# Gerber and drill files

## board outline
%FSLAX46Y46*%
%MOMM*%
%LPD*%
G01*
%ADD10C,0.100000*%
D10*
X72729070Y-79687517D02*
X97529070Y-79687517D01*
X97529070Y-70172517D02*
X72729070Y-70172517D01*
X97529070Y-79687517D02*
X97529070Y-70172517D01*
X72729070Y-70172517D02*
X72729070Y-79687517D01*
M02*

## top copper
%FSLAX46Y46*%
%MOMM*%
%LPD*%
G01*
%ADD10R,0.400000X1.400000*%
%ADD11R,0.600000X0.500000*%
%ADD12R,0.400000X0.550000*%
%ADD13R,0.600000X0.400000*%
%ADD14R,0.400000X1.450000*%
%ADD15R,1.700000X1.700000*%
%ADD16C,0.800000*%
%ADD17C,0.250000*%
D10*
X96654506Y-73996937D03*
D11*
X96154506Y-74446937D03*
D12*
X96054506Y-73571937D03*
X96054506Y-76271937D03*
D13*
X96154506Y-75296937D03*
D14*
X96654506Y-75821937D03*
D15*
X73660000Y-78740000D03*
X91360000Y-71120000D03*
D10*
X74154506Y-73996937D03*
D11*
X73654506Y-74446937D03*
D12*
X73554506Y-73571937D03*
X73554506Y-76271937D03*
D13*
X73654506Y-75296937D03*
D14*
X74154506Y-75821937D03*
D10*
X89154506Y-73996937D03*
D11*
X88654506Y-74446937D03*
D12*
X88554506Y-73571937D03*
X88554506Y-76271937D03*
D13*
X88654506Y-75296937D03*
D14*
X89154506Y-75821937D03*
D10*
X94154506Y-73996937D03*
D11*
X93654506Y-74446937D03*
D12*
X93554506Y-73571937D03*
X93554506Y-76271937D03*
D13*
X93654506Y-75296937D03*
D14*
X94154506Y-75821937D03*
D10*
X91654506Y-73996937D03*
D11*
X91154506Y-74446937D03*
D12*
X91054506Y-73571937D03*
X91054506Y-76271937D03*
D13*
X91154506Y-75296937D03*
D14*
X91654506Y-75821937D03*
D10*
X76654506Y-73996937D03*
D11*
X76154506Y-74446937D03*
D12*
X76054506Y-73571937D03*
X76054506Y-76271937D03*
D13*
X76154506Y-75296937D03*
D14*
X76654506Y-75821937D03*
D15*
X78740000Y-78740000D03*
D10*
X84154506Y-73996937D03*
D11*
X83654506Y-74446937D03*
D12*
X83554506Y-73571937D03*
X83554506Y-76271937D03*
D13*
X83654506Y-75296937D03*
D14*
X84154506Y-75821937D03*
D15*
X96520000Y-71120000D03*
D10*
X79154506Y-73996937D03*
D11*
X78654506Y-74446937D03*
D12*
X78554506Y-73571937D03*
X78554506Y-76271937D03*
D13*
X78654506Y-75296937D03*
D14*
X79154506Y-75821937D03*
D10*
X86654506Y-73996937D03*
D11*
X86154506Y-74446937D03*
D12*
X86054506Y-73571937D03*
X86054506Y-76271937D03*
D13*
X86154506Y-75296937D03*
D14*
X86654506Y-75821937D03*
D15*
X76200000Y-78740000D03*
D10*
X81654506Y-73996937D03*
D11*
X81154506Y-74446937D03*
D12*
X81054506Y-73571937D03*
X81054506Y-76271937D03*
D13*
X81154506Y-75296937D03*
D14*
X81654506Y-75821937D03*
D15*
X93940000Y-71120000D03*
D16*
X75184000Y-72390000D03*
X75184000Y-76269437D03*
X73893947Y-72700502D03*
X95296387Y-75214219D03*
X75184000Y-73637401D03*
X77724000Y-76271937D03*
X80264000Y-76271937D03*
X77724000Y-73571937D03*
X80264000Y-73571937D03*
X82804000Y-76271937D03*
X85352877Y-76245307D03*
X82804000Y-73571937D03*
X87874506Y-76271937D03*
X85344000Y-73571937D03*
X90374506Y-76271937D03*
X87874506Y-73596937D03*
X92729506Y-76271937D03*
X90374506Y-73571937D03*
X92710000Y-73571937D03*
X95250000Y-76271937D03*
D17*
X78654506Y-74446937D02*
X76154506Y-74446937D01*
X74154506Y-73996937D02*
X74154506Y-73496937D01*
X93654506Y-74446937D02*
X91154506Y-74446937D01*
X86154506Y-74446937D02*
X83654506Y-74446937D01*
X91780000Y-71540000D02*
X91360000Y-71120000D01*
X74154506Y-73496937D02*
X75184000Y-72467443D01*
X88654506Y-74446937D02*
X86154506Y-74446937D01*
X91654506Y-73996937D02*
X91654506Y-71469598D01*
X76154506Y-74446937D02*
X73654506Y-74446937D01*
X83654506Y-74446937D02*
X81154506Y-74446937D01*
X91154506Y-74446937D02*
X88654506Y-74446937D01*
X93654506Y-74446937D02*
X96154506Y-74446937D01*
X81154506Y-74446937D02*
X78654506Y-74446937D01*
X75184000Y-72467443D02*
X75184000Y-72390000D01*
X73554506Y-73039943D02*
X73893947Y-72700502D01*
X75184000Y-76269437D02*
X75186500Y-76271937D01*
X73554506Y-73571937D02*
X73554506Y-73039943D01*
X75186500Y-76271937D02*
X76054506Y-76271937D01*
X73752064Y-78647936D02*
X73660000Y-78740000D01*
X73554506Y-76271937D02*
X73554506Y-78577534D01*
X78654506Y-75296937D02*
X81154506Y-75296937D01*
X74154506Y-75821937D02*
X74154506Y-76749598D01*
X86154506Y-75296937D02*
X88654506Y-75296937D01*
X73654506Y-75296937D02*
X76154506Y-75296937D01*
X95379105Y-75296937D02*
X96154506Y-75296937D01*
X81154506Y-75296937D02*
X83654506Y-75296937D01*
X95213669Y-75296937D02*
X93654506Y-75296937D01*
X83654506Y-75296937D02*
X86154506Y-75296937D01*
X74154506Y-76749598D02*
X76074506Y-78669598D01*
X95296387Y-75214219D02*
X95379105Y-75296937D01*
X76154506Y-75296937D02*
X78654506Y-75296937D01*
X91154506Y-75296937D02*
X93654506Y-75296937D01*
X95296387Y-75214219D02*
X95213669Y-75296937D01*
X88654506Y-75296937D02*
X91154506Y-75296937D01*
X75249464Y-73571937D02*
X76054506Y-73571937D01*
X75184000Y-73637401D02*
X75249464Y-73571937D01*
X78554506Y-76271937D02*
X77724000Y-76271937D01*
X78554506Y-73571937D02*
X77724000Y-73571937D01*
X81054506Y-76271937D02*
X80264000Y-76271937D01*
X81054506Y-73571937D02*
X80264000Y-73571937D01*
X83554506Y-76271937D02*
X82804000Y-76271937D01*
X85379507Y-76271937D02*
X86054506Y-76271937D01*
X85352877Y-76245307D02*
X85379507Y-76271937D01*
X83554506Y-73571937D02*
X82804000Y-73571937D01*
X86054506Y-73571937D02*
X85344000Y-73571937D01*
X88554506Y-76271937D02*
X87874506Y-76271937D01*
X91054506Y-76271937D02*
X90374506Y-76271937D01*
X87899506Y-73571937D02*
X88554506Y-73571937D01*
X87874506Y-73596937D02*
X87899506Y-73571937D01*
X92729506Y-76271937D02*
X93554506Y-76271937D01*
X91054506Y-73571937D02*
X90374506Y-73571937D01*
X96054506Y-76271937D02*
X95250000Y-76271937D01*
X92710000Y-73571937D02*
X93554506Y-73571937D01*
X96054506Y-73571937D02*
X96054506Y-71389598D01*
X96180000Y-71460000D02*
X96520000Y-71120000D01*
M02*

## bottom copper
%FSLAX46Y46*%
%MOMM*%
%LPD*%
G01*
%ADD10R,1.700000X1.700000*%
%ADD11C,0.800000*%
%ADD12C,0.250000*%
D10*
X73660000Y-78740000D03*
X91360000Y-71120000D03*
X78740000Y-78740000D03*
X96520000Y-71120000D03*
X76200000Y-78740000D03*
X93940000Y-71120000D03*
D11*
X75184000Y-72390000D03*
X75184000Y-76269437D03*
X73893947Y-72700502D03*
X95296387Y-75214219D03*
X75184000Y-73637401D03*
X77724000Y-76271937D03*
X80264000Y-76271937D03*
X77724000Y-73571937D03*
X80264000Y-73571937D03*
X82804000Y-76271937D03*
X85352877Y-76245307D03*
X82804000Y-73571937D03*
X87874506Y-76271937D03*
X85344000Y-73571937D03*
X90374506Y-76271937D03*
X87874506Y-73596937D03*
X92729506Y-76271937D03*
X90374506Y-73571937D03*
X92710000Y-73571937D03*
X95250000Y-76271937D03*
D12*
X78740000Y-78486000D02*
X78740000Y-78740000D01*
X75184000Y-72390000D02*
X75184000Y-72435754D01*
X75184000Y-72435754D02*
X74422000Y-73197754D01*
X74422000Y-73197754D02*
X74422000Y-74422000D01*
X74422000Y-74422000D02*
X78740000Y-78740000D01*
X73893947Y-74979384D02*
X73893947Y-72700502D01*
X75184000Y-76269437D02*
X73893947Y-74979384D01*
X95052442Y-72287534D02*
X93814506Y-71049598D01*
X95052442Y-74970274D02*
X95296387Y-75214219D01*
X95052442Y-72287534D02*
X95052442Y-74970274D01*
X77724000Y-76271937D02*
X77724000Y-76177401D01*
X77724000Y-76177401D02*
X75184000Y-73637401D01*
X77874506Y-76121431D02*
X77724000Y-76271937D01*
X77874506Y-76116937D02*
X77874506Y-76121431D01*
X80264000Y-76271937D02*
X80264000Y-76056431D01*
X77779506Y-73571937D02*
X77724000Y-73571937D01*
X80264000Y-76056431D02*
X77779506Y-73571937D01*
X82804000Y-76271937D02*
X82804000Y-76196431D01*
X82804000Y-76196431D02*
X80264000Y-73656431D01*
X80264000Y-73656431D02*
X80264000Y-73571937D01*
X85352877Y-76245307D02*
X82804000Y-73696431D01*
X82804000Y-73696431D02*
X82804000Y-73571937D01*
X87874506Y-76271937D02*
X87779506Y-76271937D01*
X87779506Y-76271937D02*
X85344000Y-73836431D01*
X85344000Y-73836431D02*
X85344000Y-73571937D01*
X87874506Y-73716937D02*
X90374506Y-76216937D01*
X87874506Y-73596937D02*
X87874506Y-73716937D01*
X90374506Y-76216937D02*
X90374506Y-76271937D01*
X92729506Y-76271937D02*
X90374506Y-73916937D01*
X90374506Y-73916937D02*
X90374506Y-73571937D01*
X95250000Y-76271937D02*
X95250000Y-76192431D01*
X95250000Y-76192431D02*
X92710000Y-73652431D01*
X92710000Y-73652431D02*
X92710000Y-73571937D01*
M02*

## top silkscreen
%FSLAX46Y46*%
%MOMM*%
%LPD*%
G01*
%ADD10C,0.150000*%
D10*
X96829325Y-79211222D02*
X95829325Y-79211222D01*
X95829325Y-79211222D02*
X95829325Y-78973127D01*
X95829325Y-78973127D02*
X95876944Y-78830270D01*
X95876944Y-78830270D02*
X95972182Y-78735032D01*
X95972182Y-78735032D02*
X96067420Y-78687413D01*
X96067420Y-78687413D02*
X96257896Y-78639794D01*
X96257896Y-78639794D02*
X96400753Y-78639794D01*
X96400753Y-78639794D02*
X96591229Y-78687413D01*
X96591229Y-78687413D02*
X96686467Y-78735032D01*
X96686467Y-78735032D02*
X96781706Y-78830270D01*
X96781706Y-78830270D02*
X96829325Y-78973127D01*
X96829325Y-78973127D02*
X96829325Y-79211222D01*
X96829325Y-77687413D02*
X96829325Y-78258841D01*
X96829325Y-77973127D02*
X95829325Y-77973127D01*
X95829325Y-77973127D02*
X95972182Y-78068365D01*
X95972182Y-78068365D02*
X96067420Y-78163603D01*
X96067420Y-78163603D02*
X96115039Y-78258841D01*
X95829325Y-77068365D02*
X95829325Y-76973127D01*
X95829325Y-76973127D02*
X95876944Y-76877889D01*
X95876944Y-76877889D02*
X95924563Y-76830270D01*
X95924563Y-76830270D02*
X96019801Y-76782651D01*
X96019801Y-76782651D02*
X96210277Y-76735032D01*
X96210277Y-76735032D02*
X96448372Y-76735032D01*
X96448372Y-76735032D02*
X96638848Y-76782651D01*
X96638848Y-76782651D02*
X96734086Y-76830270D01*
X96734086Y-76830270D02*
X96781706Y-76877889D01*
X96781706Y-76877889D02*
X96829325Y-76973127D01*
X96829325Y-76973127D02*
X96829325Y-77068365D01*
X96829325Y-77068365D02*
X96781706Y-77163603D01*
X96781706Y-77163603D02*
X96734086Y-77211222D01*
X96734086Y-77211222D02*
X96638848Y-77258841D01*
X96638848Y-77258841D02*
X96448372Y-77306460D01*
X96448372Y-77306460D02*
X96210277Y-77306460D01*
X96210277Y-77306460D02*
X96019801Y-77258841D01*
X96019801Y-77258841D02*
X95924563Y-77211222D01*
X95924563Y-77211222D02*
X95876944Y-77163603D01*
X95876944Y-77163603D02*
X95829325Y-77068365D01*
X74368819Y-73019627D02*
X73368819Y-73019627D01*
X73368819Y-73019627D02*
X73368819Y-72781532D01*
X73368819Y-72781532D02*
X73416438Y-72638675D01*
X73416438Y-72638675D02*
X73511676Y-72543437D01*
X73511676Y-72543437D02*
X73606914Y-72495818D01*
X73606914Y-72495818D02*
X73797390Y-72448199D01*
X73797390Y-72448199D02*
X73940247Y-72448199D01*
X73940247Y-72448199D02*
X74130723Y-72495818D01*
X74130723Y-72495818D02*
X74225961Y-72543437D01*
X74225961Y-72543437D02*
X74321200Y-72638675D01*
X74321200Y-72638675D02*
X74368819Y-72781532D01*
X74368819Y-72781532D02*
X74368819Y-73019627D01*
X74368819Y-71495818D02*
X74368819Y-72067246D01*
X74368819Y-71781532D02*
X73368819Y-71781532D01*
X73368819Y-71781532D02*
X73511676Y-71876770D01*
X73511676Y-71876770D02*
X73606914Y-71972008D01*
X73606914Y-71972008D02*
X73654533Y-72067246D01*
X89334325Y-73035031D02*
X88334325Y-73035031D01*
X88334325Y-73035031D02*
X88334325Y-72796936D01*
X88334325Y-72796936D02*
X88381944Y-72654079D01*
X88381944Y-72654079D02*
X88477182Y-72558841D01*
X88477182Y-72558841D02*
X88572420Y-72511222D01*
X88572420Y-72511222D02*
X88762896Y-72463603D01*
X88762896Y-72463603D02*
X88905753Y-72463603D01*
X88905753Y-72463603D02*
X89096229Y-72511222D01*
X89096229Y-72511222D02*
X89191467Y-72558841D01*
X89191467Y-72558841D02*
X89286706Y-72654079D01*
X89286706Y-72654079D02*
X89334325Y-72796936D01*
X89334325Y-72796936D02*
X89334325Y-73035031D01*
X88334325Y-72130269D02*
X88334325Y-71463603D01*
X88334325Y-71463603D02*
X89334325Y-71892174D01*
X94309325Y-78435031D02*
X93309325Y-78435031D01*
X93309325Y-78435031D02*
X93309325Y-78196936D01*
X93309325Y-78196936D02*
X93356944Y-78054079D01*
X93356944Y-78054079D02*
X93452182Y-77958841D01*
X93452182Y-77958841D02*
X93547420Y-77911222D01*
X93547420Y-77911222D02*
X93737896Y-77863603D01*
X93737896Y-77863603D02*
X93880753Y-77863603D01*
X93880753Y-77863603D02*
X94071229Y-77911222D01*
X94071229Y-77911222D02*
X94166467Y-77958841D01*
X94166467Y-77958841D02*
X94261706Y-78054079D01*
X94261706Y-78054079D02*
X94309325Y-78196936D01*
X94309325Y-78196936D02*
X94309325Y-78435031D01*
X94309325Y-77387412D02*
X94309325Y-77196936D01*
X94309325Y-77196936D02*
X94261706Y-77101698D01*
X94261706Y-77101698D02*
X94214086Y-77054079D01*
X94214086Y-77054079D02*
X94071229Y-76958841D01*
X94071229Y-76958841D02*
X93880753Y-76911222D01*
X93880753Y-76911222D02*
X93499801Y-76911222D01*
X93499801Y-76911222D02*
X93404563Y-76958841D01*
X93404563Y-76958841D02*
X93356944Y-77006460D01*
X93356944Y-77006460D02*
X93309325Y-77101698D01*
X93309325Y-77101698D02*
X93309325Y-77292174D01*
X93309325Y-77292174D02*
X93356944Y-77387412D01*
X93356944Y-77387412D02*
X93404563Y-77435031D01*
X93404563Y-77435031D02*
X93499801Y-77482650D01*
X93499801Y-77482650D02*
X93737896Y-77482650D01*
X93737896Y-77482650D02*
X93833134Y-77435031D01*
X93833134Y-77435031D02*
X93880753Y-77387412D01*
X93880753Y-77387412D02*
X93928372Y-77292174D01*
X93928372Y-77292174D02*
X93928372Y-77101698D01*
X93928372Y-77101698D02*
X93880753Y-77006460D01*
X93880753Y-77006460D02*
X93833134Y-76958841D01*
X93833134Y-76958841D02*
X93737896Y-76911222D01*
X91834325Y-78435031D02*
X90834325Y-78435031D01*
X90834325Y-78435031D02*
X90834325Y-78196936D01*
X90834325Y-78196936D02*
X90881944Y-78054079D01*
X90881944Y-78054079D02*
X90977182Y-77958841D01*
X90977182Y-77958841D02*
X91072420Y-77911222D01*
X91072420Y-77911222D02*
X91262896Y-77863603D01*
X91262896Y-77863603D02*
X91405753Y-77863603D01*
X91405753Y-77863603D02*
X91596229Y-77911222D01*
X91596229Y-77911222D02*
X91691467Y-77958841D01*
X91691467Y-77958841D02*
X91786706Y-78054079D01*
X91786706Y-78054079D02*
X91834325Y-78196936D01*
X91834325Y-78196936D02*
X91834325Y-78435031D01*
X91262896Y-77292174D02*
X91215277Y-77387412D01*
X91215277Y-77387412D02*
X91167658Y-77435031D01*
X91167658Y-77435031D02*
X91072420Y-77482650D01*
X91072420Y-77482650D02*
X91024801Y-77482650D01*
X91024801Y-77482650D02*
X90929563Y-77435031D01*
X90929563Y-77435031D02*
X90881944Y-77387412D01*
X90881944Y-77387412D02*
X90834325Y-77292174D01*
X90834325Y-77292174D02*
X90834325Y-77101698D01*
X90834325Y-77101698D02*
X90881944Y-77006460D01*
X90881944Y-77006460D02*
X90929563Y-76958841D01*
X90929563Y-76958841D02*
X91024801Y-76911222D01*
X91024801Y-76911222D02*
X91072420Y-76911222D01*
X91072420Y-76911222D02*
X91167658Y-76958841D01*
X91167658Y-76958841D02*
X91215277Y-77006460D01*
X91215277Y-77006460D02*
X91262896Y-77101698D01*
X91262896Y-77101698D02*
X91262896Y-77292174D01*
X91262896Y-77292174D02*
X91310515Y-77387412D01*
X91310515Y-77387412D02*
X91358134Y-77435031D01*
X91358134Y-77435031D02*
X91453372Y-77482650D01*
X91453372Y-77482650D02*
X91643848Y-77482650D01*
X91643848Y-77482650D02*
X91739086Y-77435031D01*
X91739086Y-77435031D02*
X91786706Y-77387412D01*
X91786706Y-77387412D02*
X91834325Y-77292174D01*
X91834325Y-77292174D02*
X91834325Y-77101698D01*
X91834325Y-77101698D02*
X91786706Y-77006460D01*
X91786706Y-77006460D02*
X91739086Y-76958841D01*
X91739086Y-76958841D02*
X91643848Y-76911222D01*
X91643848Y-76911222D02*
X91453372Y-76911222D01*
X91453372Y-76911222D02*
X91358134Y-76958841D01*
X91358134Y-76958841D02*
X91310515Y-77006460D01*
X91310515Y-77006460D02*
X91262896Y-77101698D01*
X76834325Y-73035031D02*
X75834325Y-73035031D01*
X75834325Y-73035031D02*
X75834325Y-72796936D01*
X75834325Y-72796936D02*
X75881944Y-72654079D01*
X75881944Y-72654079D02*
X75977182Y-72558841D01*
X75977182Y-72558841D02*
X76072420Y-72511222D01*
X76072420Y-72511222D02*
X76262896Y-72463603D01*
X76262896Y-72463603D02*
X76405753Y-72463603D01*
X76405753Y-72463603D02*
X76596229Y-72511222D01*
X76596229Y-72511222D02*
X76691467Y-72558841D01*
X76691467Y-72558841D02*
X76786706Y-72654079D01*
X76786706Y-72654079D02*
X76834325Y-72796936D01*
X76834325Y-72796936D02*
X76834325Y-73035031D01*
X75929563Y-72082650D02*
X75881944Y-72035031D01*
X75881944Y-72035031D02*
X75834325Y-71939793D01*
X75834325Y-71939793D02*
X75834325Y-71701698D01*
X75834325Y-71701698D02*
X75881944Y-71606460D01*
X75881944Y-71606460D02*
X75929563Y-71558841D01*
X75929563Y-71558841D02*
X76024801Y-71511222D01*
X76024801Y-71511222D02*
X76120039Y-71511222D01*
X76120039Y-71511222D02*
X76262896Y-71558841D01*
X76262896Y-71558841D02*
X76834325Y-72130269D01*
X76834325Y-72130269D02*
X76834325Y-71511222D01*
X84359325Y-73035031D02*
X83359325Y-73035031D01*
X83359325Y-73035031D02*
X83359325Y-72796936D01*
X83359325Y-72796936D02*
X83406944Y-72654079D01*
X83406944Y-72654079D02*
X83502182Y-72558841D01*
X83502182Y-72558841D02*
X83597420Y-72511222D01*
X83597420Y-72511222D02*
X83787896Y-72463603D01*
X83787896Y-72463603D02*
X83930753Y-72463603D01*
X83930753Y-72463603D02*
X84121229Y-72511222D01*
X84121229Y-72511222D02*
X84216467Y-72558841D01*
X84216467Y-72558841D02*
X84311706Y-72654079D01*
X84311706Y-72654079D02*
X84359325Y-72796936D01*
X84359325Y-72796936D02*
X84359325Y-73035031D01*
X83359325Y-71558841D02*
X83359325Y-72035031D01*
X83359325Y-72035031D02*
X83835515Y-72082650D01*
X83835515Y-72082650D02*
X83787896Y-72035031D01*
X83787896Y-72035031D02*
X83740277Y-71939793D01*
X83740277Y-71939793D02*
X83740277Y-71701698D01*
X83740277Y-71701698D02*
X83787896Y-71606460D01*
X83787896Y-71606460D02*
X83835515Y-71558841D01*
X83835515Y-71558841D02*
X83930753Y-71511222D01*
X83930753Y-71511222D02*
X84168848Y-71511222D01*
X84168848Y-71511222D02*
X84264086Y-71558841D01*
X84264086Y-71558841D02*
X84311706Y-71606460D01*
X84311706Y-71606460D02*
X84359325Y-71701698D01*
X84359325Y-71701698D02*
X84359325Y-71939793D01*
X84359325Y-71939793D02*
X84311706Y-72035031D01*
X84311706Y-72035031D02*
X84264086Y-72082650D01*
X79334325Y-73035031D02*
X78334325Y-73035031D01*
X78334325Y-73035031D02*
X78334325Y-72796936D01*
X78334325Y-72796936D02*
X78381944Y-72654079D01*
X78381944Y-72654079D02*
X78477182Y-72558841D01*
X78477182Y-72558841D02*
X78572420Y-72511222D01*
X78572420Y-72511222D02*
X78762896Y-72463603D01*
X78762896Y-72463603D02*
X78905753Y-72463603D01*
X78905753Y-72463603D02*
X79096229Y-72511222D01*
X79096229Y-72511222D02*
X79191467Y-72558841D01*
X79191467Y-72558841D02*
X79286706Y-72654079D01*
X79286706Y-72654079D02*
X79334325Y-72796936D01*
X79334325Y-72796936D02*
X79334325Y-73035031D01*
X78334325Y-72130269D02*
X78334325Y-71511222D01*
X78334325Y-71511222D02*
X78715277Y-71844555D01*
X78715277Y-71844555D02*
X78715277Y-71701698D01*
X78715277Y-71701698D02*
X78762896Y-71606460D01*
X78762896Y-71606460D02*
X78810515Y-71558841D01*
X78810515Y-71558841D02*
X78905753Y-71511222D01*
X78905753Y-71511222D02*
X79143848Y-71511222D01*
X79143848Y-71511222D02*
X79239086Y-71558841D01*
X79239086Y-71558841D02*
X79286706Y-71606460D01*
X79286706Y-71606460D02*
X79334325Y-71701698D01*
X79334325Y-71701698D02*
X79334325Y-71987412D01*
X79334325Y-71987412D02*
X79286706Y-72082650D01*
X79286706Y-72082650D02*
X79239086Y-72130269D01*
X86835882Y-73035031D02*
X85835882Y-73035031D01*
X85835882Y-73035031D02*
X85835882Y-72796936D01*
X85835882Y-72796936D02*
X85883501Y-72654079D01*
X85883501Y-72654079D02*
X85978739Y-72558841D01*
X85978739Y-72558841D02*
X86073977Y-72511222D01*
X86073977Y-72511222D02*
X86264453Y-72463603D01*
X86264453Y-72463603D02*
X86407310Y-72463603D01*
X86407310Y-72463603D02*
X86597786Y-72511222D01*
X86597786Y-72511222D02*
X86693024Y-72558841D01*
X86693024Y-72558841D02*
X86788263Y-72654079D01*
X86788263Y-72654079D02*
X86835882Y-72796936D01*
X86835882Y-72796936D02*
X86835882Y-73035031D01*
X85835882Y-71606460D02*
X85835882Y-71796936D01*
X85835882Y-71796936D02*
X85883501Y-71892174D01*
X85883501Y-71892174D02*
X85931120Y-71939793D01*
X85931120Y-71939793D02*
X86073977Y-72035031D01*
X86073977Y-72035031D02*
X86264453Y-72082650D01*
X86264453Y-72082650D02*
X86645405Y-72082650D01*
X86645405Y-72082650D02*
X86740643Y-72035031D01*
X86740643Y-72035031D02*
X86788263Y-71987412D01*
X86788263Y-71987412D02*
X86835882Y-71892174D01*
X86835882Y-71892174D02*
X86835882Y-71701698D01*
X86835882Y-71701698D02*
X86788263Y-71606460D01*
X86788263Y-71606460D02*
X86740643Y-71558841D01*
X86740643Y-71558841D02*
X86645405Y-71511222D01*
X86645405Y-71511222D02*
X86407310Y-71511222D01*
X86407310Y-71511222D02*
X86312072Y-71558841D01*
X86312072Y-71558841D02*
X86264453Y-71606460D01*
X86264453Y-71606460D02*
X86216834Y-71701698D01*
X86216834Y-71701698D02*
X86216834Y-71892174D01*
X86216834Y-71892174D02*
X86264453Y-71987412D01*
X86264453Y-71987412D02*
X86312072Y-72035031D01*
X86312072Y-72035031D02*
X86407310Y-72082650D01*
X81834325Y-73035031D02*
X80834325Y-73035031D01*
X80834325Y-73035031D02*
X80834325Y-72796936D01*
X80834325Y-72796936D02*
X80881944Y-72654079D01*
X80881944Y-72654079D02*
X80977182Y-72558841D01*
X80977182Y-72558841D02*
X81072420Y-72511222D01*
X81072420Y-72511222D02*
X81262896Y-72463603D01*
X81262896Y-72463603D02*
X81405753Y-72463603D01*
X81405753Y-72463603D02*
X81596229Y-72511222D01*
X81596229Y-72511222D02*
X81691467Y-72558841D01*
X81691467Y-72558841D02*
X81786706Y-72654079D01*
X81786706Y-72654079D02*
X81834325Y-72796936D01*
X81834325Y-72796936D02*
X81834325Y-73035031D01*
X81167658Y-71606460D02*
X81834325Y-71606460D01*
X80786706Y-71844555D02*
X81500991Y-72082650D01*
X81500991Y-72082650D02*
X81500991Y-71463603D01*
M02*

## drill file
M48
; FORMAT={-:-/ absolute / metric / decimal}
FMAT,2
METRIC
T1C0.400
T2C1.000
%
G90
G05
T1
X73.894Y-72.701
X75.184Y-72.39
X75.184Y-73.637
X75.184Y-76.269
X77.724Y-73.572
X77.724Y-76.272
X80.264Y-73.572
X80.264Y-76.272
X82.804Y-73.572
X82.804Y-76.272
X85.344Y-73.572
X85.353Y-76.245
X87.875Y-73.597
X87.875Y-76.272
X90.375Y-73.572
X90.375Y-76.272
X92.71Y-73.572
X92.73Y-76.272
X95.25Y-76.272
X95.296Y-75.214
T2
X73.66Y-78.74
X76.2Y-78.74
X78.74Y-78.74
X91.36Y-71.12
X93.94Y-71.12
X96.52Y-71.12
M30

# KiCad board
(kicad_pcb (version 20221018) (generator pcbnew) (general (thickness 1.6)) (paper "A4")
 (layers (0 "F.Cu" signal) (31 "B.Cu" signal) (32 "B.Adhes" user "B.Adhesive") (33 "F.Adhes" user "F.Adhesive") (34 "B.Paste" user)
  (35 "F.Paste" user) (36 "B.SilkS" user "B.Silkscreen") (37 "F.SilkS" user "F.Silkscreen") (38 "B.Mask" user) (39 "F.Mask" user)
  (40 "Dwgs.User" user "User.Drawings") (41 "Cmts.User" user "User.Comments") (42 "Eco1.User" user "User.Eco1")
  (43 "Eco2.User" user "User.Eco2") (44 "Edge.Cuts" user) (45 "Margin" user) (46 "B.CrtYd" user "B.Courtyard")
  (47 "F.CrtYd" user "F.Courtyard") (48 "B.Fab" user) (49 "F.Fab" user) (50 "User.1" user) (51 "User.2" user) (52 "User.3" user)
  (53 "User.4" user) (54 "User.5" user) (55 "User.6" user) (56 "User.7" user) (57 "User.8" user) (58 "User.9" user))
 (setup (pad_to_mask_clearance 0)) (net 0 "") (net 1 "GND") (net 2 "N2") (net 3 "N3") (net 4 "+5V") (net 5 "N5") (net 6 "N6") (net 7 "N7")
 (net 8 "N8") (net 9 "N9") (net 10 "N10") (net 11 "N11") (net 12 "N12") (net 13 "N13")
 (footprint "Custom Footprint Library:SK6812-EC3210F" (layer "F.Cu") (at 96.354506 74.896937 -90)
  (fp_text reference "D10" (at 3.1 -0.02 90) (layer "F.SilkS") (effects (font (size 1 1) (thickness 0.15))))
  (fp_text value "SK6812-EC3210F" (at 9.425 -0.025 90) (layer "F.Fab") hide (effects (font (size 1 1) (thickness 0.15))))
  (pad "1" smd rect (at -0.9 -0.3 90) (size 1.4 0.4) (layers "F.Cu" "F.Paste" "F.Mask") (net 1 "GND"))
  (pad "1" smd rect (at -0.45 0.2 90) (size 0.5 0.6) (layers "F.Cu" "F.Paste" "F.Mask") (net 1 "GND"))
  (pad "2" smd rect (at -1.325 0.3 90) (size 0.55 0.4) (layers "F.Cu" "F.Paste" "F.Mask") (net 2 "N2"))
  (pad "3" smd rect (at 1.375 0.3 90) (size 0.55 0.4) (layers "F.Cu" "F.Paste" "F.Mask") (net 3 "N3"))
  (pad "4" smd rect (at 0.4 0.2 90) (size 0.4 0.6) (layers "F.Cu" "F.Paste" "F.Mask") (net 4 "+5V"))
  (pad "4" smd rect (at 0.925 -0.3 90) (size 1.45 0.4) (layers "F.Cu" "F.Paste" "F.Mask") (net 4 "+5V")))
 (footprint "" (layer "F.Cu") (at 73.66 78.74)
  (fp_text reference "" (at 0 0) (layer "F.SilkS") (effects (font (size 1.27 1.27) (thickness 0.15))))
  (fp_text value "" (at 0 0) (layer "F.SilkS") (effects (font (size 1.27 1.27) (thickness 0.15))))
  (pad "1" thru_hole rect (at 0 0) (size 1.7 1.7) (drill 1) (layers "*.Cu" "*.Mask") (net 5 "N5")))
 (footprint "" (layer "F.Cu") (at 91.44 71.12)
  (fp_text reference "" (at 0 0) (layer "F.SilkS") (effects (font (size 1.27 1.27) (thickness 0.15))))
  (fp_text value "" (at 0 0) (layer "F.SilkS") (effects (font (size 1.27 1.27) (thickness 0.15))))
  (pad "1" thru_hole rect (at -0.08 0) (size 1.7 1.7) (drill 1) (layers "*.Cu" "*.Mask") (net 1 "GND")))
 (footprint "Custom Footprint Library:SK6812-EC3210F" (layer "F.Cu") (at 73.854506 74.896937 -90)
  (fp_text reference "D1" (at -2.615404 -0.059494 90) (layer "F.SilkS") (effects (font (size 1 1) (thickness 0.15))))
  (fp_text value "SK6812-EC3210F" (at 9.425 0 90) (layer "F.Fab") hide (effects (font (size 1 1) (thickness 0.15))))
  (pad "1" smd rect (at -0.9 -0.3 90) (size 1.4 0.4) (layers "F.Cu" "F.Paste" "F.Mask") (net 1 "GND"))
  (pad "1" smd rect (at -0.45 0.2 90) (size 0.5 0.6) (layers "F.Cu" "F.Paste" "F.Mask") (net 1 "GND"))
  (pad "2" smd rect (at -1.325 0.3 90) (size 0.55 0.4) (layers "F.Cu" "F.Paste" "F.Mask") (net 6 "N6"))
  (pad "3" smd rect (at 1.375 0.3 90) (size 0.55 0.4) (layers "F.Cu" "F.Paste" "F.Mask") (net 5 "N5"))
  (pad "4" smd rect (at 0.4 0.2 90) (size 0.4 0.6) (layers "F.Cu" "F.Paste" "F.Mask") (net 4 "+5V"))
  (pad "4" smd rect (at 0.925 -0.3 90) (size 1.45 0.4) (layers "F.Cu" "F.Paste" "F.Mask") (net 4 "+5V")))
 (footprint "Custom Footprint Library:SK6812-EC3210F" (layer "F.Cu") (at 88.854506 74.896937 -90)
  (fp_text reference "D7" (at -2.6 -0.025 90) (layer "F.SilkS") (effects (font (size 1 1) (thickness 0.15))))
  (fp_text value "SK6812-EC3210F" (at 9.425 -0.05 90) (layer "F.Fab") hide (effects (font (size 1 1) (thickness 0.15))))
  (pad "1" smd rect (at -0.9 -0.3 90) (size 1.4 0.4) (layers "F.Cu" "F.Paste" "F.Mask") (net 1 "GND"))
  (pad "1" smd rect (at -0.45 0.2 90) (size 0.5 0.6) (layers "F.Cu" "F.Paste" "F.Mask") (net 1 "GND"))
  (pad "2" smd rect (at -1.325 0.3 90) (size 0.55 0.4) (layers "F.Cu" "F.Paste" "F.Mask") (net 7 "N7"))
  (pad "3" smd rect (at 1.375 0.3 90) (size 0.55 0.4) (layers "F.Cu" "F.Paste" "F.Mask") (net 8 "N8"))
  (pad "4" smd rect (at 0.4 0.2 90) (size 0.4 0.6) (layers "F.Cu" "F.Paste" "F.Mask") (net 4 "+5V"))
  (pad "4" smd rect (at 0.925 -0.3 90) (size 1.45 0.4) (layers "F.Cu" "F.Paste" "F.Mask") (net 4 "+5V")))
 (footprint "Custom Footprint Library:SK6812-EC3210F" (layer "F.Cu") (at 93.854506 74.896937 -90)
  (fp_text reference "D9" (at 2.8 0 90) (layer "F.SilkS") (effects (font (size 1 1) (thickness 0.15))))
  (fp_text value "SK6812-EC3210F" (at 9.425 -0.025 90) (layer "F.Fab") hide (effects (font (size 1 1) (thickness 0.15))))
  (pad "1" smd rect (at -0.9 -0.3 90) (size 1.4 0.4) (layers "F.Cu" "F.Paste" "F.Mask") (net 1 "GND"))
  (pad "1" smd rect (at -0.45 0.2 90) (size 0.5 0.6) (layers "F.Cu" "F.Paste" "F.Mask") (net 1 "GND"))
  (pad "2" smd rect (at -1.325 0.3 90) (size 0.55 0.4) (layers "F.Cu" "F.Paste" "F.Mask") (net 3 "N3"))
  (pad "3" smd rect (at 1.375 0.3 90) (size 0.55 0.4) (layers "F.Cu" "F.Paste" "F.Mask") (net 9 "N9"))
  (pad "4" smd rect (at 0.4 0.2 90) (size 0.4 0.6) (layers "F.Cu" "F.Paste" "F.Mask") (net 4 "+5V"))
  (pad "4" smd rect (at 0.925 -0.3 90) (size 1.45 0.4) (layers "F.Cu" "F.Paste" "F.Mask") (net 4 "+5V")))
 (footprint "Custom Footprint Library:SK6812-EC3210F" (layer "F.Cu") (at 91.354506 74.896937 -90)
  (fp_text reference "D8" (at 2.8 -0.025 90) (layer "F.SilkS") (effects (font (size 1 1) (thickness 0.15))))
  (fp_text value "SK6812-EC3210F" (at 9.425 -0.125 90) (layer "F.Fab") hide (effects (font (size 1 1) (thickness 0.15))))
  (pad "1" smd rect (at -0.9 -0.3 90) (size 1.4 0.4) (layers "F.Cu" "F.Paste" "F.Mask") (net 1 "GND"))
  (pad "1" smd rect (at -0.45 0.2 90) (size 0.5 0.6) (layers "F.Cu" "F.Paste" "F.Mask") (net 1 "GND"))
  (pad "2" smd rect (at -1.325 0.3 90) (size 0.55 0.4) (layers "F.Cu" "F.Paste" "F.Mask") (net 9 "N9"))
  (pad "3" smd rect (at 1.375 0.3 90) (size 0.55 0.4) (layers "F.Cu" "F.Paste" "F.Mask") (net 7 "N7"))
  (pad "4" smd rect (at 0.4 0.2 90) (size 0.4 0.6) (layers "F.Cu" "F.Paste" "F.Mask") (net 4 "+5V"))
  (pad "4" smd rect (at 0.925 -0.3 90) (size 1.45 0.4) (layers "F.Cu" "F.Paste" "F.Mask") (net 4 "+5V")))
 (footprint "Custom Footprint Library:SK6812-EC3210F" (layer "F.Cu") (at 76.354506 74.896937 -90)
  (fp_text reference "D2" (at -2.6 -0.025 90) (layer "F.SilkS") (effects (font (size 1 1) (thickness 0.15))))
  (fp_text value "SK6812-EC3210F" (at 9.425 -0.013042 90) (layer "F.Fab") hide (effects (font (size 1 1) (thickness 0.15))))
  (pad "1" smd rect (at -0.9 -0.3 90) (size 1.4 0.4) (layers "F.Cu" "F.Paste" "F.Mask") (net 1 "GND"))
  (pad "1" smd rect (at -0.45 0.2 90) (size 0.5 0.6) (layers "F.Cu" "F.Paste" "F.Mask") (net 1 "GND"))
  (pad "2" smd rect (at -1.325 0.3 90) (size 0.55 0.4) (layers "F.Cu" "F.Paste" "F.Mask") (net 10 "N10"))
  (pad "3" smd rect (at 1.375 0.3 90) (size 0.55 0.4) (layers "F.Cu" "F.Paste" "F.Mask") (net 6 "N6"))
  (pad "4" smd rect (at 0.4 0.2 90) (size 0.4 0.6) (layers "F.Cu" "F.Paste" "F.Mask") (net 4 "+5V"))
  (pad "4" smd rect (at 0.925 -0.3 90) (size 1.45 0.4) (layers "F.Cu" "F.Paste" "F.Mask") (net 4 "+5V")))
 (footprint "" (layer "F.Cu") (at 78.74 78.74)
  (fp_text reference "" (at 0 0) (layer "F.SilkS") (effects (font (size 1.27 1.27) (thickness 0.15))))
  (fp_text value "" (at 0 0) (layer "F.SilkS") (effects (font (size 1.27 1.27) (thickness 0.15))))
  (pad "1" thru_hole rect (at 0 0) (size 1.7 1.7) (drill 1) (layers "*.Cu" "*.Mask") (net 1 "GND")))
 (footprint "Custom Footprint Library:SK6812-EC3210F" (layer "F.Cu") (at 83.854506 74.896937 -90)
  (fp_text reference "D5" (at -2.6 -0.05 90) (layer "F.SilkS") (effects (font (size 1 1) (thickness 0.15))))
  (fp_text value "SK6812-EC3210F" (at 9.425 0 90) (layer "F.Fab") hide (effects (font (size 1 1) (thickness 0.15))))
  (pad "1" smd rect (at -0.9 -0.3 90) (size 1.4 0.4) (layers "F.Cu" "F.Paste" "F.Mask") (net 1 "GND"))
  (pad "1" smd rect (at -0.45 0.2 90) (size 0.5 0.6) (layers "F.Cu" "F.Paste" "F.Mask") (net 1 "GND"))
  (pad "2" smd rect (at -1.325 0.3 90) (size 0.55 0.4) (layers "F.Cu" "F.Paste" "F.Mask") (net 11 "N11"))
  (pad "3" smd rect (at 1.375 0.3 90) (size 0.55 0.4) (layers "F.Cu" "F.Paste" "F.Mask") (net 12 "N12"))
  (pad "4" smd rect (at 0.4 0.2 90) (size 0.4 0.6) (layers "F.Cu" "F.Paste" "F.Mask") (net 4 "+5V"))
  (pad "4" smd rect (at 0.925 -0.3 90) (size 1.45 0.4) (layers "F.Cu" "F.Paste" "F.Mask") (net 4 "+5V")))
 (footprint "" (layer "F.Cu") (at 96.52 71.12)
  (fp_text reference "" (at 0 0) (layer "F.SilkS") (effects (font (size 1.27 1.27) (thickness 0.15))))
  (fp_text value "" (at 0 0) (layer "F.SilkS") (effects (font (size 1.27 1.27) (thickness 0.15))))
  (pad "1" thru_hole rect (at 0 0) (size 1.7 1.7) (drill 1) (layers "*.Cu" "*.Mask") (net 2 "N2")))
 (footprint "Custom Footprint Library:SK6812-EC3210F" (layer "F.Cu") (at 78.854506 74.896937 -90)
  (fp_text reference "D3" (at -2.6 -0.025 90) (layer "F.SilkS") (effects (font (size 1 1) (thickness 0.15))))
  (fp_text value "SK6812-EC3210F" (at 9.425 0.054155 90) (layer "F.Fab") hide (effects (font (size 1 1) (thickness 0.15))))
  (pad "1" smd rect (at -0.9 -0.3 90) (size 1.4 0.4) (layers "F.Cu" "F.Paste" "F.Mask") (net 1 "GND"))
  (pad "1" smd rect (at -0.45 0.2 90) (size 0.5 0.6) (layers "F.Cu" "F.Paste" "F.Mask") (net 1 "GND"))
  (pad "2" smd rect (at -1.325 0.3 90) (size 0.55 0.4) (layers "F.Cu" "F.Paste" "F.Mask") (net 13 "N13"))
  (pad "3" smd rect (at 1.375 0.3 90) (size 0.55 0.4) (layers "F.Cu" "F.Paste" "F.Mask") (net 10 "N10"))
  (pad "4" smd rect (at 0.4 0.2 90) (size 0.4 0.6) (layers "F.Cu" "F.Paste" "F.Mask") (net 4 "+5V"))
  (pad "4" smd rect (at 0.925 -0.3 90) (size 1.45 0.4) (layers "F.Cu" "F.Paste" "F.Mask") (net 4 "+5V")))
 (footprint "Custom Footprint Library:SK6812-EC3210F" (layer "F.Cu") (at 86.354506 74.896937 -90)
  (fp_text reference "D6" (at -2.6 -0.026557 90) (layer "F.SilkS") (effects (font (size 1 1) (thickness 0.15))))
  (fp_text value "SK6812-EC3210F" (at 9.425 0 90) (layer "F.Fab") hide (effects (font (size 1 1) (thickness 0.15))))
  (pad "1" smd rect (at -0.9 -0.3 90) (size 1.4 0.4) (layers "F.Cu" "F.Paste" "F.Mask") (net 1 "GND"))
  (pad "1" smd rect (at -0.45 0.2 90) (size 0.5 0.6) (layers "F.Cu" "F.Paste" "F.Mask") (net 1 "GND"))
  (pad "2" smd rect (at -1.325 0.3 90) (size 0.55 0.4) (layers "F.Cu" "F.Paste" "F.Mask") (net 8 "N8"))
  (pad "3" smd rect (at 1.375 0.3 90) (size 0.55 0.4) (layers "F.Cu" "F.Paste" "F.Mask") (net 11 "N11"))
  (pad "4" smd rect (at 0.4 0.2 90) (size 0.4 0.6) (layers "F.Cu" "F.Paste" "F.Mask") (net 4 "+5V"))
  (pad "4" smd rect (at 0.925 -0.3 90) (size 1.45 0.4) (layers "F.Cu" "F.Paste" "F.Mask") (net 4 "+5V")))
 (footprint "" (layer "F.Cu") (at 76.2 78.74)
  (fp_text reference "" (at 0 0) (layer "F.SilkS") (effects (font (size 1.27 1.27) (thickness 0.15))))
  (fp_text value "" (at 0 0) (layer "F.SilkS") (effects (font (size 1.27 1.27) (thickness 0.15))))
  (pad "1" thru_hole rect (at 0 0) (size 1.7 1.7) (drill 1) (layers "*.Cu" "*.Mask") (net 4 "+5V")))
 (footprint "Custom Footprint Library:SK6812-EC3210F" (layer "F.Cu") (at 81.354506 74.896937 -90)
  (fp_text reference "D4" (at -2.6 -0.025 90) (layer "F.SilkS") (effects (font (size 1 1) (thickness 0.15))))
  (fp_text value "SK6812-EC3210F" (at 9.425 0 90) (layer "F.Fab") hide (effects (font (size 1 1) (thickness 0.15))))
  (pad "1" smd rect (at -0.9 -0.3 90) (size 1.4 0.4) (layers "F.Cu" "F.Paste" "F.Mask") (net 1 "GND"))
  (pad "1" smd rect (at -0.45 0.2 90) (size 0.5 0.6) (layers "F.Cu" "F.Paste" "F.Mask") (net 1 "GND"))
  (pad "2" smd rect (at -1.325 0.3 90) (size 0.55 0.4) (layers "F.Cu" "F.Paste" "F.Mask") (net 12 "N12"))
  (pad "3" smd rect (at 1.375 0.3 90) (size 0.55 0.4) (layers "F.Cu" "F.Paste" "F.Mask") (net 13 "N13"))
  (pad "4" smd rect (at 0.4 0.2 90) (size 0.4 0.6) (layers "F.Cu" "F.Paste" "F.Mask") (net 4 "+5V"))
  (pad "4" smd rect (at 0.925 -0.3 90) (size 1.45 0.4) (layers "F.Cu" "F.Paste" "F.Mask") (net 4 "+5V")))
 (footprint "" (layer "F.Cu") (at 93.98 71.12)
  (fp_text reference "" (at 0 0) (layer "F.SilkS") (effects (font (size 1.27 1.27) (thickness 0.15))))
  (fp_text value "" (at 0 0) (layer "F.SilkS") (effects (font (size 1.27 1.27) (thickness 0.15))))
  (pad "1" thru_hole rect (at -0.04 0) (size 1.7 1.7) (drill 1) (layers "*.Cu" "*.Mask") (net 4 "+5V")))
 (gr_line (start 72.72907 79.687517) (end 97.52907 79.687517) (stroke (width 0.1) (type solid)) (layer "Edge.Cuts"))
 (gr_line (start 97.52907 70.172517) (end 72.72907 70.172517) (stroke (width 0.1) (type solid)) (layer "Edge.Cuts"))
 (gr_line (start 97.52907 79.687517) (end 97.52907 70.172517) (stroke (width 0.1) (type solid)) (layer "Edge.Cuts"))
 (gr_line (start 72.72907 70.172517) (end 72.72907 79.687517) (stroke (width 0.1) (type solid)) (layer "Edge.Cuts"))
 (segment (start 78.654506 74.446937) (end 76.154506 74.446937) (width 0.25) (layer "F.Cu") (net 1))
 (segment (start 74.154506 73.996937) (end 74.154506 73.496937) (width 0.25) (layer "F.Cu") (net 1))
 (segment (start 93.654506 74.446937) (end 91.154506 74.446937) (width 0.25) (layer "F.Cu") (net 1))
 (segment (start 86.154506 74.446937) (end 83.654506 74.446937) (width 0.25) (layer "F.Cu") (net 1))
 (segment (start 91.78 71.54) (end 91.36 71.12) (width 0.25) (layer "F.Cu") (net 1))
 (segment (start 74.154506 73.496937) (end 75.184 72.467443) (width 0.25) (layer "F.Cu") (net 1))
 (segment (start 88.654506 74.446937) (end 86.154506 74.446937) (width 0.25) (layer "F.Cu") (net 1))
 (segment (start 91.654506 73.996937) (end 91.654506 71.469598) (width 0.25) (layer "F.Cu") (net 1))
 (segment (start 76.154506 74.446937) (end 73.654506 74.446937) (width 0.25) (layer "F.Cu") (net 1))
 (segment (start 83.654506 74.446937) (end 81.154506 74.446937) (width 0.25) (layer "F.Cu") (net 1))
 (segment (start 91.154506 74.446937) (end 88.654506 74.446937) (width 0.25) (layer "F.Cu") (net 1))
 (segment (start 93.654506 74.446937) (end 96.154506 74.446937) (width 0.25) (layer "F.Cu") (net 1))
 (segment (start 81.154506 74.446937) (end 78.654506 74.446937) (width 0.25) (layer "F.Cu") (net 1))
 (segment (start 75.184 72.467443) (end 75.184 72.39) (width 0.25) (layer "F.Cu") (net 1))
 (via (at 75.184 72.39) (size 0.8) (drill 0.4) (layers "F.Cu" "B.Cu") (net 1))
 (segment (start 78.74 78.486) (end 78.74 78.74) (width 0.25) (layer "B.Cu") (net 1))
 (segment (start 75.184 72.39) (end 75.184 72.435754) (width 0.25) (layer "B.Cu") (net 1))
 (segment (start 75.184 72.435754) (end 74.422 73.197754) (width 0.25) (layer "B.Cu") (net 1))
 (segment (start 74.422 73.197754) (end 74.422 74.422) (width 0.25) (layer "B.Cu") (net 1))
 (segment (start 74.422 74.422) (end 78.74 78.74) (width 0.25) (layer "B.Cu") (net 1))
 (segment (start 73.554506 73.039943) (end 73.893947 72.700502) (width 0.25) (layer "F.Cu") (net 6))
 (segment (start 75.184 76.269437) (end 75.1865 76.271937) (width 0.25) (layer "F.Cu") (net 6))
 (segment (start 73.554506 73.571937) (end 73.554506 73.039943) (width 0.25) (layer "F.Cu") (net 6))
 (segment (start 75.1865 76.271937) (end 76.054506 76.271937) (width 0.25) (layer "F.Cu") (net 6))
 (via (at 75.184 76.269437) (size 0.8) (drill 0.4) (layers "F.Cu" "B.Cu") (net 6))
 (via (at 73.893947 72.700502) (size 0.8) (drill 0.4) (layers "F.Cu" "B.Cu") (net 6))
 (segment (start 73.893947 74.979384) (end 73.893947 72.700502) (width 0.25) (layer "B.Cu") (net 6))
 (segment (start 75.184 76.269437) (end 73.893947 74.979384) (width 0.25) (layer "B.Cu") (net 6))
 (segment (start 73.752064 78.647936) (end 73.66 78.74) (width 0.25) (layer "F.Cu") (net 5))
 (segment (start 73.554506 76.271937) (end 73.554506 78.577534) (width 0.25) (layer "F.Cu") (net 5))
 (segment (start 78.654506 75.296937) (end 81.154506 75.296937) (width 0.25) (layer "F.Cu") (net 4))
 (segment (start 74.154506 75.821937) (end 74.154506 76.749598) (width 0.25) (layer "F.Cu") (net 4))
 (segment (start 86.154506 75.296937) (end 88.654506 75.296937) (width 0.25) (layer "F.Cu") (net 4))
 (segment (start 73.654506 75.296937) (end 76.154506 75.296937) (width 0.25) (layer "F.Cu") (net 4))
 (segment (start 95.379105 75.296937) (end 96.154506 75.296937) (width 0.25) (layer "F.Cu") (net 4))
 (segment (start 81.154506 75.296937) (end 83.654506 75.296937) (width 0.25) (layer "F.Cu") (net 4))
 (segment (start 95.213669 75.296937) (end 93.654506 75.296937) (width 0.25) (layer "F.Cu") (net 4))
 (segment (start 83.654506 75.296937) (end 86.154506 75.296937) (width 0.25) (layer "F.Cu") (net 4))
 (segment (start 74.154506 76.749598) (end 76.074506 78.669598) (width 0.25) (layer "F.Cu") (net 4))
 (segment (start 95.296387 75.214219) (end 95.379105 75.296937) (width 0.25) (layer "F.Cu") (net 4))
 (segment (start 76.154506 75.296937) (end 78.654506 75.296937) (width 0.25) (layer "F.Cu") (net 4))
 (segment (start 91.154506 75.296937) (end 93.654506 75.296937) (width 0.25) (layer "F.Cu") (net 4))
 (segment (start 95.296387 75.214219) (end 95.213669 75.296937) (width 0.25) (layer "F.Cu") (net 4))
 (segment (start 88.654506 75.296937) (end 91.154506 75.296937) (width 0.25) (layer "F.Cu") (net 4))
 (via (at 95.296387 75.214219) (size 0.8) (drill 0.4) (layers "F.Cu" "B.Cu") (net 4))
 (segment (start 95.052442 72.287534) (end 93.814506 71.049598) (width 0.25) (layer "B.Cu") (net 4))
 (segment (start 95.052442 74.970274) (end 95.296387 75.214219) (width 0.25) (layer "B.Cu") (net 4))
 (segment (start 95.052442 72.287534) (end 95.052442 74.970274) (width 0.25) (layer "B.Cu") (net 4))
 (segment (start 75.249464 73.571937) (end 76.054506 73.571937) (width 0.25) (layer "F.Cu") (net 10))
 (segment (start 75.184 73.637401) (end 75.249464 73.571937) (width 0.25) (layer "F.Cu") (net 10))
 (segment (start 78.554506 76.271937) (end 77.724 76.271937) (width 0.25) (layer "F.Cu") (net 10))
 (via (at 75.184 73.637401) (size 0.8) (drill 0.4) (layers "F.Cu" "B.Cu") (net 10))
 (via (at 77.724 76.271937) (size 0.8) (drill 0.4) (layers "F.Cu" "B.Cu") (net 10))
 (segment (start 77.724 76.271937) (end 77.724 76.177401) (width 0.25) (layer "B.Cu") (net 10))
 (segment (start 77.724 76.177401) (end 75.184 73.637401) (width 0.25) (layer "B.Cu") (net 10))
 (segment (start 77.874506 76.121431) (end 77.724 76.271937) (width 0.25) (layer "B.Cu") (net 10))
 (segment (start 77.874506 76.116937) (end 77.874506 76.121431) (width 0.25) (layer "B.Cu") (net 10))
 (segment (start 78.554506 73.571937) (end 77.724 73.571937) (width 0.25) (layer "F.Cu") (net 13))
 (segment (start 81.054506 76.271937) (end 80.264 76.271937) (width 0.25) (layer "F.Cu") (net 13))
 (via (at 80.264 76.271937) (size 0.8) (drill 0.4) (layers "F.Cu" "B.Cu") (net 13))
 (via (at 77.724 73.571937) (size 0.8) (drill 0.4) (layers "F.Cu" "B.Cu") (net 13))
 (segment (start 80.264 76.271937) (end 80.264 76.056431) (width 0.25) (layer "B.Cu") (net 13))
 (segment (start 77.779506 73.571937) (end 77.724 73.571937) (width 0.25) (layer "B.Cu") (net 13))
 (segment (start 80.264 76.056431) (end 77.779506 73.571937) (width 0.25) (layer "B.Cu") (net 13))
 (segment (start 81.054506 73.571937) (end 80.264 73.571937) (width 0.25) (layer "F.Cu") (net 12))
 (segment (start 83.554506 76.271937) (end 82.804 76.271937) (width 0.25) (layer "F.Cu") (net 12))
 (via (at 80.264 73.571937) (size 0.8) (drill 0.4) (layers "F.Cu" "B.Cu") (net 12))
 (via (at 82.804 76.271937) (size 0.8) (drill 0.4) (layers "F.Cu" "B.Cu") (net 12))
 (segment (start 82.804 76.271937) (end 82.804 76.196431) (width 0.25) (layer "B.Cu") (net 12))
 (segment (start 82.804 76.196431) (end 80.264 73.656431) (width 0.25) (layer "B.Cu") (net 12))
 (segment (start 80.264 73.656431) (end 80.264 73.571937) (width 0.25) (layer "B.Cu") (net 12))
 (segment (start 85.379507 76.271937) (end 86.054506 76.271937) (width 0.25) (layer "F.Cu") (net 11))
 (segment (start 85.352877 76.245307) (end 85.379507 76.271937) (width 0.25) (layer "F.Cu") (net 11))
 (segment (start 83.554506 73.571937) (end 82.804 73.571937) (width 0.25) (layer "F.Cu") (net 11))
 (via (at 85.352877 76.245307) (size 0.8) (drill 0.4) (layers "F.Cu" "B.Cu") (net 11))
 (via (at 82.804 73.571937) (size 0.8) (drill 0.4) (layers "F.Cu" "B.Cu") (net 11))
 (segment (start 85.352877 76.245307) (end 82.804 73.696431) (width 0.25) (layer "B.Cu") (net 11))
 (segment (start 82.804 73.696431) (end 82.804 73.571937) (width 0.25) (layer "B.Cu") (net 11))
 (segment (start 86.054506 73.571937) (end 85.344 73.571937) (width 0.25) (layer "F.Cu") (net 8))
 (segment (start 88.554506 76.271937) (end 87.874506 76.271937) (width 0.25) (layer "F.Cu") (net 8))
 (via (at 87.874506 76.271937) (size 0.8) (drill 0.4) (layers "F.Cu" "B.Cu") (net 8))
 (via (at 85.344 73.571937) (size 0.8) (drill 0.4) (layers "F.Cu" "B.Cu") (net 8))
 (segment (start 87.874506 76.271937) (end 87.779506 76.271937) (width 0.25) (layer "B.Cu") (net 8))
 (segment (start 87.779506 76.271937) (end 85.344 73.836431) (width 0.25) (layer "B.Cu") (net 8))
 (segment (start 85.344 73.836431) (end 85.344 73.571937) (width 0.25) (layer "B.Cu") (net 8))
 (segment (start 91.054506 76.271937) (end 90.374506 76.271937) (width 0.25) (layer "F.Cu") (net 7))
 (segment (start 87.899506 73.571937) (end 88.554506 73.571937) (width 0.25) (layer "F.Cu") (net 7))
 (segment (start 87.874506 73.596937) (end 87.899506 73.571937) (width 0.25) (layer "F.Cu") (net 7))
 (via (at 90.374506 76.271937) (size 0.8) (drill 0.4) (layers "F.Cu" "B.Cu") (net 7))
 (via (at 87.874506 73.596937) (size 0.8) (drill 0.4) (layers "F.Cu" "B.Cu") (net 7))
 (segment (start 87.874506 73.716937) (end 90.374506 76.216937) (width 0.25) (layer "B.Cu") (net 7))
 (segment (start 87.874506 73.596937) (end 87.874506 73.716937) (width 0.25) (layer "B.Cu") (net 7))
 (segment (start 90.374506 76.216937) (end 90.374506 76.271937) (width 0.25) (layer "B.Cu") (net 7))
 (segment (start 92.729506 76.271937) (end 93.554506 76.271937) (width 0.25) (layer "F.Cu") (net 9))
 (segment (start 91.054506 73.571937) (end 90.374506 73.571937) (width 0.25) (layer "F.Cu") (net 9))
 (via (at 92.729506 76.271937) (size 0.8) (drill 0.4) (layers "F.Cu" "B.Cu") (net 9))
 (via (at 90.374506 73.571937) (size 0.8) (drill 0.4) (layers "F.Cu" "B.Cu") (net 9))
 (segment (start 92.729506 76.271937) (end 90.374506 73.916937) (width 0.25) (layer "B.Cu") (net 9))
 (segment (start 90.374506 73.916937) (end 90.374506 73.571937) (width 0.25) (layer "B.Cu") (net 9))
 (segment (start 96.054506 76.271937) (end 95.25 76.271937) (width 0.25) (layer "F.Cu") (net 3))
 (segment (start 92.71 73.571937) (end 93.554506 73.571937) (width 0.25) (layer "F.Cu") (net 3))
 (via (at 92.71 73.571937) (size 0.8) (drill 0.4) (layers "F.Cu" "B.Cu") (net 3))
 (via (at 95.25 76.271937) (size 0.8) (drill 0.4) (layers "F.Cu" "B.Cu") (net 3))
 (segment (start 95.25 76.271937) (end 95.25 76.192431) (width 0.25) (layer "B.Cu") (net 3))
 (segment (start 95.25 76.192431) (end 92.71 73.652431) (width 0.25) (layer "B.Cu") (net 3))
 (segment (start 92.71 73.652431) (end 92.71 73.571937) (width 0.25) (layer "B.Cu") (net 3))
 (segment (start 96.054506 73.571937) (end 96.054506 71.389598) (width 0.25) (layer "F.Cu") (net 2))
 (segment (start 96.18 71.46) (end 96.52 71.12) (width 0.25) (layer "F.Cu") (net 2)))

